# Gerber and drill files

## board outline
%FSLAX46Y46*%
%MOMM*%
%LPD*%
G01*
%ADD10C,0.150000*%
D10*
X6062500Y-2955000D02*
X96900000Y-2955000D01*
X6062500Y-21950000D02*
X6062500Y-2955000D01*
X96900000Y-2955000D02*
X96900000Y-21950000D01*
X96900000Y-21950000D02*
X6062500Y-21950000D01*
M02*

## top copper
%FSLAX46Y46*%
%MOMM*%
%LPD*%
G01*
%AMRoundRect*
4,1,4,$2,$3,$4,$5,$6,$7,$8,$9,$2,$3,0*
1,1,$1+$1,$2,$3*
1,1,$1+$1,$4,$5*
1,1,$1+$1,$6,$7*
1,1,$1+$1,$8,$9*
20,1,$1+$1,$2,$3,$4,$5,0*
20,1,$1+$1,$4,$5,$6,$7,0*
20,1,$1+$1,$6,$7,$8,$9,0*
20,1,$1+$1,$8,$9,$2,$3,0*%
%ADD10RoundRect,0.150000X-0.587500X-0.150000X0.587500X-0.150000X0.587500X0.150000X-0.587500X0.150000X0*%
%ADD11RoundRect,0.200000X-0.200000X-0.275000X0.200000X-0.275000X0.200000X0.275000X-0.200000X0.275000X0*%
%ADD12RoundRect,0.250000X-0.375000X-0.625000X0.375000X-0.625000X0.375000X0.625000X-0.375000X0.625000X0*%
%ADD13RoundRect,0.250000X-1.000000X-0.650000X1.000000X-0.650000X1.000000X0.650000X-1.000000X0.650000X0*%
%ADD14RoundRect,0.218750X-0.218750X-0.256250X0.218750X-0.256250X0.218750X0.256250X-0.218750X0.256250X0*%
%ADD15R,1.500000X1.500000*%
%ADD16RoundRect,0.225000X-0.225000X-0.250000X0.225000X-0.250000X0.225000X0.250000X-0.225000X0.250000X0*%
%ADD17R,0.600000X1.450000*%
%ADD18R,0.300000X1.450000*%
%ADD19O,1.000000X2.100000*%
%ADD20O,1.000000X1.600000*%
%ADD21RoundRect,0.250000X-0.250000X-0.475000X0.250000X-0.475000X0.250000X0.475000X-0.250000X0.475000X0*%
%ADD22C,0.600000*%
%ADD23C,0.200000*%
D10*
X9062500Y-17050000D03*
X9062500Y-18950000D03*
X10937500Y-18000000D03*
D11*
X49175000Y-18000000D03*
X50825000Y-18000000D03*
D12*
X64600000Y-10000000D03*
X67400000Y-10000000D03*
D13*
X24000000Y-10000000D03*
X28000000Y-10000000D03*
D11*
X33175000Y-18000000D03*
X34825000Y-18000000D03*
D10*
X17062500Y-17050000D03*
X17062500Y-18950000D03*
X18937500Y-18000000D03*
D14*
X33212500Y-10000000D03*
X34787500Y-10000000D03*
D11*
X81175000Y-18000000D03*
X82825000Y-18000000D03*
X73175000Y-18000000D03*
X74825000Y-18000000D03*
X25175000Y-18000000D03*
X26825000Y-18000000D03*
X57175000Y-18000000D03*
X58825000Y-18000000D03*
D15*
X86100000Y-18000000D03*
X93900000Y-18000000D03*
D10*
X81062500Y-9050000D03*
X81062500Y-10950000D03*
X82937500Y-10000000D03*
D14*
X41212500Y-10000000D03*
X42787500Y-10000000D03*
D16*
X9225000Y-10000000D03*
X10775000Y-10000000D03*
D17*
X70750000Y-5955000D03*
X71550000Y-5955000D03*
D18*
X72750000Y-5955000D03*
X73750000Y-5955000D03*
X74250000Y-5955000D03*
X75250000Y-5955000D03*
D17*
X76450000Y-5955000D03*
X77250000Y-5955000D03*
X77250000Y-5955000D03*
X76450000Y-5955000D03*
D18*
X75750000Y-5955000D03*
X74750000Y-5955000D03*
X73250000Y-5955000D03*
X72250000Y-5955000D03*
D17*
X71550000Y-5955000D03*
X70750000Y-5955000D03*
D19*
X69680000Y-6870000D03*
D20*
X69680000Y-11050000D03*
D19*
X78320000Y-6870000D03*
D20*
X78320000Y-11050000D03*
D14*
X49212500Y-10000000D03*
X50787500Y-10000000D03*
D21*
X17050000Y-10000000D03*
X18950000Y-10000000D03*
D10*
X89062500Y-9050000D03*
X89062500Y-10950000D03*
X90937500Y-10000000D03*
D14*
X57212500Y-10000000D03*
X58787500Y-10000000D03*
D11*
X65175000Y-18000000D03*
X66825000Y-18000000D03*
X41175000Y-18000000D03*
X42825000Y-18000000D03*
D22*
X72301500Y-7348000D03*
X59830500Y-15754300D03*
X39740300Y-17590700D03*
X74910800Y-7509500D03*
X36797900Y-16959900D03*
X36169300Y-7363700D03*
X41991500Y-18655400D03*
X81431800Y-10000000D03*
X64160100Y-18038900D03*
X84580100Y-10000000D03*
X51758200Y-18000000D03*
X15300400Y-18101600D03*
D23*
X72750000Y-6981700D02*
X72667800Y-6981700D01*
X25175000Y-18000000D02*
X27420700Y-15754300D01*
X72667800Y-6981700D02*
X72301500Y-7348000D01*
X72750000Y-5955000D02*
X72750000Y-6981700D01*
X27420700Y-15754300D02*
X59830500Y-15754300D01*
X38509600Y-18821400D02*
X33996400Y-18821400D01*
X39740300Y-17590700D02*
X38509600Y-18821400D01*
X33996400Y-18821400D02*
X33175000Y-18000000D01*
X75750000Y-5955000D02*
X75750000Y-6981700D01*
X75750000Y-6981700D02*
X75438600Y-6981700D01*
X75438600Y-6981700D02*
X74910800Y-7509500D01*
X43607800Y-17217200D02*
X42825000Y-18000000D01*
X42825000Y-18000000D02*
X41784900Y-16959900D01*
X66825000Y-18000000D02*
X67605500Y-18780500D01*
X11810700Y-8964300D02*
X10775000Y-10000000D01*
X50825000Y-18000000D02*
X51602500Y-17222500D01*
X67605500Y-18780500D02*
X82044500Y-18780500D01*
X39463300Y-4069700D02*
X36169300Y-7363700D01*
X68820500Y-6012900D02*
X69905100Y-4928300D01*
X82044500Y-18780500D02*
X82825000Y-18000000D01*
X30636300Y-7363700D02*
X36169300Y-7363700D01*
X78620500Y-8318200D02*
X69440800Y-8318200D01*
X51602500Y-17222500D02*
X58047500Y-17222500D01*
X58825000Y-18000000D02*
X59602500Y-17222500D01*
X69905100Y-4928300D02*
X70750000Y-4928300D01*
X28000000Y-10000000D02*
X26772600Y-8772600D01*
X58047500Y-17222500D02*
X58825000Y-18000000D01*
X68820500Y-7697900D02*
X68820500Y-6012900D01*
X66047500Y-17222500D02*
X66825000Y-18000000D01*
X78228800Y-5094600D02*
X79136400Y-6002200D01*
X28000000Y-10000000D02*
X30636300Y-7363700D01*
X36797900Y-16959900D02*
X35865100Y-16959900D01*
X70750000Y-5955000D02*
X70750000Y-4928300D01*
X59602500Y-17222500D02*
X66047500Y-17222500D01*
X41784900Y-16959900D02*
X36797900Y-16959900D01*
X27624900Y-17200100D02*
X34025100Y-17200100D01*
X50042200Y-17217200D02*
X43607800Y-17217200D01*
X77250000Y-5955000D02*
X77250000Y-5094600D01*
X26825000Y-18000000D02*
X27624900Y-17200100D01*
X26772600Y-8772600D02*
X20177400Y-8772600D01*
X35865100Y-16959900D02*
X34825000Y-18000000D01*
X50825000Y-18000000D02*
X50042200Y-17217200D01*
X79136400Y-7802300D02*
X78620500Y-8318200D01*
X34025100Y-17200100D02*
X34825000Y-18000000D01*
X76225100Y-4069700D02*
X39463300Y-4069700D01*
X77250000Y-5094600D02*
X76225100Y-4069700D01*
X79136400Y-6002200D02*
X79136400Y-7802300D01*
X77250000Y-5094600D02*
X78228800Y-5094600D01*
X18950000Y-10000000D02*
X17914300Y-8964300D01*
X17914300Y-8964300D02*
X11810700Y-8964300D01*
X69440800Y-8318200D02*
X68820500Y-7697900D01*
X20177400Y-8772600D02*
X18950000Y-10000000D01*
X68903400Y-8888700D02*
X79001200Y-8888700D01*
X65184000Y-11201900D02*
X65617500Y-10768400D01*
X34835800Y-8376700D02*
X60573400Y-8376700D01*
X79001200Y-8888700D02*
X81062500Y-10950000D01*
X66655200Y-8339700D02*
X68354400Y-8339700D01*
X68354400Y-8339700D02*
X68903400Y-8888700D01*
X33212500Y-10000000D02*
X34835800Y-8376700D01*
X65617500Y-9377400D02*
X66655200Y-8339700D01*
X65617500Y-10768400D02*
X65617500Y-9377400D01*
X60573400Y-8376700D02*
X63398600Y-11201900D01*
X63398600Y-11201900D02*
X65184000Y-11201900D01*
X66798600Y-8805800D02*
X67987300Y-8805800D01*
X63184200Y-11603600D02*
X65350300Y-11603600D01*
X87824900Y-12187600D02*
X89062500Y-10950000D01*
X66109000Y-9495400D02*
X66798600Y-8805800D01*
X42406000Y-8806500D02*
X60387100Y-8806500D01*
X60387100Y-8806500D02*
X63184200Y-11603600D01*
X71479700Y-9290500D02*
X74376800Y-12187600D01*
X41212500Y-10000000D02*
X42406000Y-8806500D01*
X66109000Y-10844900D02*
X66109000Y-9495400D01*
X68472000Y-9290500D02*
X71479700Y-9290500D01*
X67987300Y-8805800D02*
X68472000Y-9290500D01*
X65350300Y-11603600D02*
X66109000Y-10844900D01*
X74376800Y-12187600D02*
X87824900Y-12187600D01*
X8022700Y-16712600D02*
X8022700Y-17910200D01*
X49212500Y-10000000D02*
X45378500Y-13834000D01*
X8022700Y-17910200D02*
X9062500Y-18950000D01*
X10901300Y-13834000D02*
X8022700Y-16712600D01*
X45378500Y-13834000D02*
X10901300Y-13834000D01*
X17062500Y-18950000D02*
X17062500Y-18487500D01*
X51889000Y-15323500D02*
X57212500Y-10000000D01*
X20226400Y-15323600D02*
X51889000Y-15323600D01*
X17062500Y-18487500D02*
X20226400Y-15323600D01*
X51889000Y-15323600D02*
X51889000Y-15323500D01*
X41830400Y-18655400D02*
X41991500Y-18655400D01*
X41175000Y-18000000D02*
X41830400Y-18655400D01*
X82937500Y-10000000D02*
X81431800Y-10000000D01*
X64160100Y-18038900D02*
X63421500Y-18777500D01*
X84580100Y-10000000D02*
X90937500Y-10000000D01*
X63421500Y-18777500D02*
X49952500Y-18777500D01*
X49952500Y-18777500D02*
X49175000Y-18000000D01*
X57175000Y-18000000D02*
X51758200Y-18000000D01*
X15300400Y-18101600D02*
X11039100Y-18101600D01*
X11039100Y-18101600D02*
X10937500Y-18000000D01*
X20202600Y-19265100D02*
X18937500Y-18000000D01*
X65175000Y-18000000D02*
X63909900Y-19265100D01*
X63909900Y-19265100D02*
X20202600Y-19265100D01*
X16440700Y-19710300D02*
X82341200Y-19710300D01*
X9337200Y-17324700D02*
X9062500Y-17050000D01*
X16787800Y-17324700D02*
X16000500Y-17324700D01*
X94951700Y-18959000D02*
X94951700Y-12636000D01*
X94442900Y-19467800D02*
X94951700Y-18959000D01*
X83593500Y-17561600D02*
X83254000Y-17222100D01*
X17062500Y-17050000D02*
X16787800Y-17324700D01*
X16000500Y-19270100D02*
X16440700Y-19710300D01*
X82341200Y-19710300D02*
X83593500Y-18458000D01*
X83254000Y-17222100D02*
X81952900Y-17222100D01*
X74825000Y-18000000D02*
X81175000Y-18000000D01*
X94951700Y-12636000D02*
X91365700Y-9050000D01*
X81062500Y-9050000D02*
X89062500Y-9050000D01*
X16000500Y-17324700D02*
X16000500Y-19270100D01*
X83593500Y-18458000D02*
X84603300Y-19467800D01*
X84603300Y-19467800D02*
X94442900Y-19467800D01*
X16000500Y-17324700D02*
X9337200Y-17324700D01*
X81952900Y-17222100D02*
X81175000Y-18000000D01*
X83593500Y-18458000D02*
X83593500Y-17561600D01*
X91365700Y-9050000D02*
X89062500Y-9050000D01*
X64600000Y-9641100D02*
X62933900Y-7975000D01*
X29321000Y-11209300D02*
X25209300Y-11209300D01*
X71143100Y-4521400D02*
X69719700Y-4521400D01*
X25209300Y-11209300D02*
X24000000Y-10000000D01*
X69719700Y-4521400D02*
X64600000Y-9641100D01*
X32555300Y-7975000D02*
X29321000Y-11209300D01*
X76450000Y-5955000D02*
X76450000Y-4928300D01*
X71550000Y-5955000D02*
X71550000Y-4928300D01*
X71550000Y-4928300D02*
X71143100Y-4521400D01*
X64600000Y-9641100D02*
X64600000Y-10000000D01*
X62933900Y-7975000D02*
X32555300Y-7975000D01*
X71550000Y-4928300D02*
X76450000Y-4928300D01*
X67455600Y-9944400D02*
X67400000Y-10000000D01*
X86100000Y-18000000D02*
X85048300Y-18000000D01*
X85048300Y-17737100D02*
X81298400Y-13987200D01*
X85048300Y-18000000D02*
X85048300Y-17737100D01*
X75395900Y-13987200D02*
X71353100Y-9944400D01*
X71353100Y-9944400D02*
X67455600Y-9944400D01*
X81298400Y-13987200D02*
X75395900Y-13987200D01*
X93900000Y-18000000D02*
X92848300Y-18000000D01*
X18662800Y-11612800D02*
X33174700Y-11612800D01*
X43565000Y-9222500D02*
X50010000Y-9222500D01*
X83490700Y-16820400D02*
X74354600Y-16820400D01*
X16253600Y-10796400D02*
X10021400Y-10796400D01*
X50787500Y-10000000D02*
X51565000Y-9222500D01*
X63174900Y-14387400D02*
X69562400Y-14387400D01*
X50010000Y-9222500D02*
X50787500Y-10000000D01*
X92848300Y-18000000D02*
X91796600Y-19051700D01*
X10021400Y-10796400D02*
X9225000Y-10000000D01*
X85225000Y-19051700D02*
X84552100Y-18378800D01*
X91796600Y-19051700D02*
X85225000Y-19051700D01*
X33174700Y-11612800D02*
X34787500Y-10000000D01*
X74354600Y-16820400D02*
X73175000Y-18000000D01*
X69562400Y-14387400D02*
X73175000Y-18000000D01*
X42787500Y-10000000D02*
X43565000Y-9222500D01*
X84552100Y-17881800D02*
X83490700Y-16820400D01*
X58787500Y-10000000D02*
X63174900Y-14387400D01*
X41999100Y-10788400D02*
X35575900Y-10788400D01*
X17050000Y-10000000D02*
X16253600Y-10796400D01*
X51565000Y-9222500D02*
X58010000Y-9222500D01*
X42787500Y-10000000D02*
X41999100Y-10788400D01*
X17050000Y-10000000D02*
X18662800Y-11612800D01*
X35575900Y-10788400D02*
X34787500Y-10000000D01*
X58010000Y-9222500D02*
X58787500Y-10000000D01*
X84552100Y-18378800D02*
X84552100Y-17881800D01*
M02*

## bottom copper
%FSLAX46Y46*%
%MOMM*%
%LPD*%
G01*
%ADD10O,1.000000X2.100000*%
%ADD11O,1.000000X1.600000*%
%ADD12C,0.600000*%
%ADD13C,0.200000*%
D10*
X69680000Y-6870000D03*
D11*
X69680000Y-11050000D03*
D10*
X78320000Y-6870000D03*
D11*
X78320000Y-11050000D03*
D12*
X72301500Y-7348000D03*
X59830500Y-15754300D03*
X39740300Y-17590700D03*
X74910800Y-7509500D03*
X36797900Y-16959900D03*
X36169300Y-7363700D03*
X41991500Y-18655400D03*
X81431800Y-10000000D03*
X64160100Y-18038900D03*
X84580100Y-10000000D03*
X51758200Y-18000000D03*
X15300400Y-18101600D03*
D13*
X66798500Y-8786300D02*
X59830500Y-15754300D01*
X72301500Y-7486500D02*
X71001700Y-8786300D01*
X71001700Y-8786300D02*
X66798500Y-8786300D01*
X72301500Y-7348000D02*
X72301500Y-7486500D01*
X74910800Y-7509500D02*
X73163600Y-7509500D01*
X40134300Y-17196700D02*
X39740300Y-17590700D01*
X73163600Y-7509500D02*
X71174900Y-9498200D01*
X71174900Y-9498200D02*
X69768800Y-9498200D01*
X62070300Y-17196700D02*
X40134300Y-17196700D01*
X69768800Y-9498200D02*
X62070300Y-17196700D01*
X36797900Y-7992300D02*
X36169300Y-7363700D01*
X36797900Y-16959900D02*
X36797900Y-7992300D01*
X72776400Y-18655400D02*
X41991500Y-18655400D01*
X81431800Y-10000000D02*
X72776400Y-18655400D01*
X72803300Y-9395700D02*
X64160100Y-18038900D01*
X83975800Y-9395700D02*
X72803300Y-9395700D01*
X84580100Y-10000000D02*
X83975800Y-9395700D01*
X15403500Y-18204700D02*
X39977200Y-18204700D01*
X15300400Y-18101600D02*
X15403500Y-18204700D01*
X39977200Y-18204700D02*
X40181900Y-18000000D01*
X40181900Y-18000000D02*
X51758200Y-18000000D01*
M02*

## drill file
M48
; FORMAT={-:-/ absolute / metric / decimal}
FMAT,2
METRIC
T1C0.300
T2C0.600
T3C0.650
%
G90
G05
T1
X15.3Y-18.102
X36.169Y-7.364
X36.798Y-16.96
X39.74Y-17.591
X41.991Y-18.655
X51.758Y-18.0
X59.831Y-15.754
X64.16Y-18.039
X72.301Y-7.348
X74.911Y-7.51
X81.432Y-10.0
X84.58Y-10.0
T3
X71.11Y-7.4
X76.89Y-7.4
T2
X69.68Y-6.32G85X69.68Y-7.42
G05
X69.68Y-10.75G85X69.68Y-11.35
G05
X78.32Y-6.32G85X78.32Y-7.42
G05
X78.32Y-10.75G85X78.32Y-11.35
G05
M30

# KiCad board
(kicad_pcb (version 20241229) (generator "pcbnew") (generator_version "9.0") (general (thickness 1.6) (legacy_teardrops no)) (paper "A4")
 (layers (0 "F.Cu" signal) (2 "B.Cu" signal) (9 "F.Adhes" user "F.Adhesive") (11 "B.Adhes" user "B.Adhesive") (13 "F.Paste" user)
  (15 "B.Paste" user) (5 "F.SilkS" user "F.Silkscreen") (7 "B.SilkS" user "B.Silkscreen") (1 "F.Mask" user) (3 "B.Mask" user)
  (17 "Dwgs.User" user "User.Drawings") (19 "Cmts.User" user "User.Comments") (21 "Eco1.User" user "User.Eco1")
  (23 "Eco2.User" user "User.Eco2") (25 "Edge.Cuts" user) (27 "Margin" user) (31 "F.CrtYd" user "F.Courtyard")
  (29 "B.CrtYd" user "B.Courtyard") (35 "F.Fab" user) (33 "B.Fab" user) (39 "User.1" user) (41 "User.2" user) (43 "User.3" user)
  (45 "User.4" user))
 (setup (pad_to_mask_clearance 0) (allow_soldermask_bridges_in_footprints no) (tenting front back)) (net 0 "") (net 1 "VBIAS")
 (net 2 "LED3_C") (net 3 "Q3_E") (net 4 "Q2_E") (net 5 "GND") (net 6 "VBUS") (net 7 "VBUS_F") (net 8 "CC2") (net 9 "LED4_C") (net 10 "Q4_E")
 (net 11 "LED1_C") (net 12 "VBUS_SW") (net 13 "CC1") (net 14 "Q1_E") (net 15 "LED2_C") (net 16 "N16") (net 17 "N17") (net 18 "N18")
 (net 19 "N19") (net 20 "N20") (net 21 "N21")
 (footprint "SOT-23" (layer "F.Cu") (at 10 18)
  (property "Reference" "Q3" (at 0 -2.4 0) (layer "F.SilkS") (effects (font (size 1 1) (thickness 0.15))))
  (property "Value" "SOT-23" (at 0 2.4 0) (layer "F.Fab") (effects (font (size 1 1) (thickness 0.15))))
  (pad "1" smd roundrect (at -0.9375 -0.95) (size 1.475 0.6) (layers "F.Cu" "F.Mask" "F.Paste") (roundrect_rratio 0.25) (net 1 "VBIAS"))
  (pad "2" smd roundrect (at -0.9375 0.95) (size 1.475 0.6) (layers "F.Cu" "F.Mask" "F.Paste") (roundrect_rratio 0.25) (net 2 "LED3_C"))
  (pad "3" smd roundrect (at 0.9375 0) (size 1.475 0.6) (layers "F.Cu" "F.Mask" "F.Paste") (roundrect_rratio 0.25) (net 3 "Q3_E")))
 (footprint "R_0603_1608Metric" (layer "F.Cu") (at 50 18)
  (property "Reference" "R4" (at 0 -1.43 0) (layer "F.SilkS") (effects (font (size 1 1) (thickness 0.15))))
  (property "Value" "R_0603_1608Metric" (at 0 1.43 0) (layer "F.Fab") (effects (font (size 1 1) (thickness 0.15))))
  (pad "1" smd roundrect (at -0.825 0) (size 0.8 0.95) (layers "F.Cu" "F.Mask" "F.Paste") (roundrect_rratio 0.25) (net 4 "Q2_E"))
  (pad "2" smd roundrect (at 0.825 0) (size 0.8 0.95) (layers "F.Cu" "F.Mask" "F.Paste") (roundrect_rratio 0.25) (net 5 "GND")))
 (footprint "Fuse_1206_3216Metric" (layer "F.Cu") (at 66 10)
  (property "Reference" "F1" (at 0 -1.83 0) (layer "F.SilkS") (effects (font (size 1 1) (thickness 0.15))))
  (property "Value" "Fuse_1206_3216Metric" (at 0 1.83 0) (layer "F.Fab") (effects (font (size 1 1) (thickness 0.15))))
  (pad "1" smd roundrect (at -1.4 0) (size 1.25 1.75) (layers "F.Cu" "F.Mask" "F.Paste") (roundrect_rratio 0.2) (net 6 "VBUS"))
  (pad "2" smd roundrect (at 1.4 0) (size 1.25 1.75) (layers "F.Cu" "F.Mask" "F.Paste") (roundrect_rratio 0.2) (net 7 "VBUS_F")))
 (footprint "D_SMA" (layer "F.Cu") (at 26 10)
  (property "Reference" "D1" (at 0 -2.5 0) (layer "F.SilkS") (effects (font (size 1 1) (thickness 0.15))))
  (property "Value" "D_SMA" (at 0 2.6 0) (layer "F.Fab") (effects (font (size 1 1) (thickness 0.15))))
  (pad "1" smd roundrect (at -2 0) (size 2.5 1.8) (layers "F.Cu" "F.Mask" "F.Paste") (roundrect_rratio 0.1388888889) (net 6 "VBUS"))
  (pad "2" smd roundrect (at 2 0) (size 2.5 1.8) (layers "F.Cu" "F.Mask" "F.Paste") (roundrect_rratio 0.1388888889) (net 5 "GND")))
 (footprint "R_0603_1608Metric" (layer "F.Cu") (at 34 18)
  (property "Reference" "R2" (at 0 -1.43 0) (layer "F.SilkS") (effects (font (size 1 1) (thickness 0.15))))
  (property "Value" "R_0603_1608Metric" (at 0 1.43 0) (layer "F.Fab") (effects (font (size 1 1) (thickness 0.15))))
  (pad "1" smd roundrect (at -0.825 0) (size 0.8 0.95) (layers "F.Cu" "F.Mask" "F.Paste") (roundrect_rratio 0.25) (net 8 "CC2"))
  (pad "2" smd roundrect (at 0.825 0) (size 0.8 0.95) (layers "F.Cu" "F.Mask" "F.Paste") (roundrect_rratio 0.25) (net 5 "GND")))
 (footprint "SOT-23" (layer "F.Cu") (at 18 18)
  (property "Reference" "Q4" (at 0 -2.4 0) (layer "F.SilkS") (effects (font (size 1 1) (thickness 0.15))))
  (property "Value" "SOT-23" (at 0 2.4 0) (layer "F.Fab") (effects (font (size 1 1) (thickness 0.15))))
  (pad "1" smd roundrect (at -0.9375 -0.95) (size 1.475 0.6) (layers "F.Cu" "F.Mask" "F.Paste") (roundrect_rratio 0.25) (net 1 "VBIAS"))
  (pad "2" smd roundrect (at -0.9375 0.95) (size 1.475 0.6) (layers "F.Cu" "F.Mask" "F.Paste") (roundrect_rratio 0.25) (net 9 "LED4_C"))
  (pad "3" smd roundrect (at 0.9375 0) (size 1.475 0.6) (layers "F.Cu" "F.Mask" "F.Paste") (roundrect_rratio 0.25) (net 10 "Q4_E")))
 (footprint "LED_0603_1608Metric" (layer "F.Cu") (at 34 10)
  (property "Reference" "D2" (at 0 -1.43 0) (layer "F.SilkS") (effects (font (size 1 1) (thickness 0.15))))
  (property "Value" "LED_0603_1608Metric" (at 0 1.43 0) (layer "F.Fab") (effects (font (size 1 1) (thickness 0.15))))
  (pad "1" smd roundrect (at -0.7875 0) (size 0.875 0.95) (layers "F.Cu" "F.Mask" "F.Paste") (roundrect_rratio 0.25) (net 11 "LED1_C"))
  (pad "2" smd roundrect (at 0.7875 0) (size 0.875 0.95) (layers "F.Cu" "F.Mask" "F.Paste") (roundrect_rratio 0.25) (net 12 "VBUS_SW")))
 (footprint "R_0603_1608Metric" (layer "F.Cu") (at 82 18)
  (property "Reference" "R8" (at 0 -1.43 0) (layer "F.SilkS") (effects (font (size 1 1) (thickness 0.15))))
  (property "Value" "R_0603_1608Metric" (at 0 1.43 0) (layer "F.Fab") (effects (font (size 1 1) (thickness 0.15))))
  (pad "1" smd roundrect (at -0.825 0) (size 0.8 0.95) (layers "F.Cu" "F.Mask" "F.Paste") (roundrect_rratio 0.25) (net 1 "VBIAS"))
  (pad "2" smd roundrect (at 0.825 0) (size 0.8 0.95) (layers "F.Cu" "F.Mask" "F.Paste") (roundrect_rratio 0.25) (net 5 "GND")))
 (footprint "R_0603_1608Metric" (layer "F.Cu") (at 74 18)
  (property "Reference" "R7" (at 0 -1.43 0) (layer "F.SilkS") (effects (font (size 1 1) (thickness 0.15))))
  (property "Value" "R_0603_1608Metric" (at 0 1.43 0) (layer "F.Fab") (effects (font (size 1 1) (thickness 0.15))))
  (pad "1" smd roundrect (at -0.825 0) (size 0.8 0.95) (layers "F.Cu" "F.Mask" "F.Paste") (roundrect_rratio 0.25) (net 12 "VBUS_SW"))
  (pad "2" smd roundrect (at 0.825 0) (size 0.8 0.95) (layers "F.Cu" "F.Mask" "F.Paste") (roundrect_rratio 0.25) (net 1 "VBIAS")))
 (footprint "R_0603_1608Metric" (layer "F.Cu") (at 26 18)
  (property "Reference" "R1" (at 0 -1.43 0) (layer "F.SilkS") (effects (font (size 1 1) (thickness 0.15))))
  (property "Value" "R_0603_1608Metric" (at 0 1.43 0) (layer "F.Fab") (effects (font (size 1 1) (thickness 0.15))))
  (pad "1" smd roundrect (at -0.825 0) (size 0.8 0.95) (layers "F.Cu" "F.Mask" "F.Paste") (roundrect_rratio 0.25) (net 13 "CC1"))
  (pad "2" smd roundrect (at 0.825 0) (size 0.8 0.95) (layers "F.Cu" "F.Mask" "F.Paste") (roundrect_rratio 0.25) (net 5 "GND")))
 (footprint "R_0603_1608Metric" (layer "F.Cu") (at 58 18)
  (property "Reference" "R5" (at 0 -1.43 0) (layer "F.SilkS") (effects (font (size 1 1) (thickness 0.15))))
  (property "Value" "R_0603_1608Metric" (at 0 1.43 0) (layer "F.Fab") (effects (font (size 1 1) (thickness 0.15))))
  (pad "1" smd roundrect (at -0.825 0) (size 0.8 0.95) (layers "F.Cu" "F.Mask" "F.Paste") (roundrect_rratio 0.25) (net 3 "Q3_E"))
  (pad "2" smd roundrect (at 0.825 0) (size 0.8 0.95) (layers "F.Cu" "F.Mask" "F.Paste") (roundrect_rratio 0.25) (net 5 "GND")))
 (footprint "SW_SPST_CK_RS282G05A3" (layer "F.Cu") (at 90 18)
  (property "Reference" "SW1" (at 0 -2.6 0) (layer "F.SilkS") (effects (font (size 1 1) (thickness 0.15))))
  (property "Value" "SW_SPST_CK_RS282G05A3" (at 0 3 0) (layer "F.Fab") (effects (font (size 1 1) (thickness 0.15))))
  (pad "1" smd rect (at -3.9 0) (size 1.5 1.5) (layers "F.Cu" "F.Mask" "F.Paste") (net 7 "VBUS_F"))
  (pad "2" smd rect (at 3.9 0) (size 1.5 1.5) (layers "F.Cu" "F.Mask" "F.Paste") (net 12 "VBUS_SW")))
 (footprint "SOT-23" (layer "F.Cu") (at 82 10)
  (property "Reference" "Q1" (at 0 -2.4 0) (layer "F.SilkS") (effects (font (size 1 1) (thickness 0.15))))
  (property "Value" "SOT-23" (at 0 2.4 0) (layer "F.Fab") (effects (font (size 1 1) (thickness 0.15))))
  (pad "1" smd roundrect (at -0.9375 -0.95) (size 1.475 0.6) (layers "F.Cu" "F.Mask" "F.Paste") (roundrect_rratio 0.25) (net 1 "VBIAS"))
  (pad "2" smd roundrect (at -0.9375 0.95) (size 1.475 0.6) (layers "F.Cu" "F.Mask" "F.Paste") (roundrect_rratio 0.25) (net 11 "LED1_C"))
  (pad "3" smd roundrect (at 0.9375 0) (size 1.475 0.6) (layers "F.Cu" "F.Mask" "F.Paste") (roundrect_rratio 0.25) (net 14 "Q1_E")))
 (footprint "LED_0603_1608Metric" (layer "F.Cu") (at 42 10)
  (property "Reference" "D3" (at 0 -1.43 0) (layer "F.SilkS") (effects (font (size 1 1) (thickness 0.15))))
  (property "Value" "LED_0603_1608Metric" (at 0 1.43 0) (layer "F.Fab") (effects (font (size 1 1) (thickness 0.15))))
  (pad "1" smd roundrect (at -0.7875 0) (size 0.875 0.95) (layers "F.Cu" "F.Mask" "F.Paste") (roundrect_rratio 0.25) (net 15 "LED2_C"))
  (pad "2" smd roundrect (at 0.7875 0) (size 0.875 0.95) (layers "F.Cu" "F.Mask" "F.Paste") (roundrect_rratio 0.25) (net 12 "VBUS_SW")))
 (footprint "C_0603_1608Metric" (layer "F.Cu") (at 10 10)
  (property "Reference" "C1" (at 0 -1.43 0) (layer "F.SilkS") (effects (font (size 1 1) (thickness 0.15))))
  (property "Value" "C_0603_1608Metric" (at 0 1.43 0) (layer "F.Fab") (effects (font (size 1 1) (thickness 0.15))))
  (pad "1" smd roundrect (at -0.775 0) (size 0.9 0.95) (layers "F.Cu" "F.Mask" "F.Paste") (roundrect_rratio 0.25) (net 12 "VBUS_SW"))
  (pad "2" smd roundrect (at 0.775 0) (size 0.9 0.95) (layers "F.Cu" "F.Mask" "F.Paste") (roundrect_rratio 0.25) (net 5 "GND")))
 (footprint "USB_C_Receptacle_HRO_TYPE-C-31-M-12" (layer "F.Cu") (at 74 10)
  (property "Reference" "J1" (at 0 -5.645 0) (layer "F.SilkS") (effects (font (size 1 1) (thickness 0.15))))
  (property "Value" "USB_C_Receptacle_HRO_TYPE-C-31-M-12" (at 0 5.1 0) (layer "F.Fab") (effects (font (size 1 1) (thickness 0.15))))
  (pad "" np_thru_hole circle (at -2.89 -2.6) (size 0.65 0.65) (drill 0.65) (layers "*.Cu" "*.Mask"))
  (pad "" np_thru_hole circle (at 2.89 -2.6) (size 0.65 0.65) (drill 0.65) (layers "*.Cu" "*.Mask"))
  (pad "A1" smd rect (at -3.25 -4.045) (size 0.6 1.45) (layers "F.Cu" "F.Mask" "F.Paste") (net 5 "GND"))
  (pad "A4" smd rect (at -2.45 -4.045) (size 0.6 1.45) (layers "F.Cu" "F.Mask" "F.Paste") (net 6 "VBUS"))
  (pad "A5" smd rect (at -1.25 -4.045) (size 0.3 1.45) (layers "F.Cu" "F.Mask" "F.Paste") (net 13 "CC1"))
  (pad "A6" smd rect (at -0.25 -4.045) (size 0.3 1.45) (layers "F.Cu" "F.Mask" "F.Paste") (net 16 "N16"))
  (pad "A7" smd rect (at 0.25 -4.045) (size 0.3 1.45) (layers "F.Cu" "F.Mask" "F.Paste") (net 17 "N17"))
  (pad "A8" smd rect (at 1.25 -4.045) (size 0.3 1.45) (layers "F.Cu" "F.Mask" "F.Paste") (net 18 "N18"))
  (pad "A9" smd rect (at 2.45 -4.045) (size 0.6 1.45) (layers "F.Cu" "F.Mask" "F.Paste") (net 6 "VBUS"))
  (pad "A12" smd rect (at 3.25 -4.045) (size 0.6 1.45) (layers "F.Cu" "F.Mask" "F.Paste") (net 5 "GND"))
  (pad "B1" smd rect (at 3.25 -4.045) (size 0.6 1.45) (layers "F.Cu" "F.Mask" "F.Paste") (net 5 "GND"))
  (pad "B4" smd rect (at 2.45 -4.045) (size 0.6 1.45) (layers "F.Cu" "F.Mask" "F.Paste") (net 6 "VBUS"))
  (pad "B5" smd rect (at 1.75 -4.045) (size 0.3 1.45) (layers "F.Cu" "F.Mask" "F.Paste") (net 8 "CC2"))
  (pad "B6" smd rect (at 0.75 -4.045) (size 0.3 1.45) (layers "F.Cu" "F.Mask" "F.Paste") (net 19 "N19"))
  (pad "B7" smd rect (at -0.75 -4.045) (size 0.3 1.45) (layers "F.Cu" "F.Mask" "F.Paste") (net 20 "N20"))
  (pad "B8" smd rect (at -1.75 -4.045) (size 0.3 1.45) (layers "F.Cu" "F.Mask" "F.Paste") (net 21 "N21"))
  (pad "B9" smd rect (at -2.45 -4.045) (size 0.6 1.45) (layers "F.Cu" "F.Mask" "F.Paste") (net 6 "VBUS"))
  (pad "B12" smd rect (at -3.25 -4.045) (size 0.6 1.45) (layers "F.Cu" "F.Mask" "F.Paste") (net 5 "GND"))
  (pad "S1" thru_hole oval (at -4.32 -3.13) (size 1 2.1) (drill oval 0.6 1.7) (layers "*.Cu" "*.Mask") (remove_unused_layers no))
  (pad "S1" thru_hole oval (at -4.32 1.05) (size 1 1.6) (drill oval 0.6 1.2) (layers "*.Cu" "*.Mask") (remove_unused_layers no))
  (pad "S1" thru_hole oval (at 4.32 -3.13) (size 1 2.1) (drill oval 0.6 1.7) (layers "*.Cu" "*.Mask") (remove_unused_layers no))
  (pad "S1" thru_hole oval (at 4.32 1.05) (size 1 1.6) (drill oval 0.6 1.2) (layers "*.Cu" "*.Mask") (remove_unused_layers no)))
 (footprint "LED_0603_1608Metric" (layer "F.Cu") (at 50 10)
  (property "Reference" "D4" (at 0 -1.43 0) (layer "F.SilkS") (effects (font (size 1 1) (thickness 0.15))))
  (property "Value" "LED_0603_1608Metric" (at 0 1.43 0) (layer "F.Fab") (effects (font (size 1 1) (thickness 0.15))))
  (pad "1" smd roundrect (at -0.7875 0) (size 0.875 0.95) (layers "F.Cu" "F.Mask" "F.Paste") (roundrect_rratio 0.25) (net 2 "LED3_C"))
  (pad "2" smd roundrect (at 0.7875 0) (size 0.875 0.95) (layers "F.Cu" "F.Mask" "F.Paste") (roundrect_rratio 0.25) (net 12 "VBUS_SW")))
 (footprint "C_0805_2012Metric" (layer "F.Cu") (at 18 10)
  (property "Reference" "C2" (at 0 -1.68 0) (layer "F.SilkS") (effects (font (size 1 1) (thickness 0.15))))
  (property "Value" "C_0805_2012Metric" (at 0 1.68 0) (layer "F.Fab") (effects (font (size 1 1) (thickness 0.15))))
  (pad "1" smd roundrect (at -0.95 0) (size 1 1.45) (layers "F.Cu" "F.Mask" "F.Paste") (roundrect_rratio 0.25) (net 12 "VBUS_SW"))
  (pad "2" smd roundrect (at 0.95 0) (size 1 1.45) (layers "F.Cu" "F.Mask" "F.Paste") (roundrect_rratio 0.25) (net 5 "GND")))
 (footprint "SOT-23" (layer "F.Cu") (at 90 10)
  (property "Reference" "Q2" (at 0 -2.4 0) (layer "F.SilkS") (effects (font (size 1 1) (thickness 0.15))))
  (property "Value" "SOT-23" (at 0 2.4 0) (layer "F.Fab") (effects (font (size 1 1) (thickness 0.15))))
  (pad "1" smd roundrect (at -0.9375 -0.95) (size 1.475 0.6) (layers "F.Cu" "F.Mask" "F.Paste") (roundrect_rratio 0.25) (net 1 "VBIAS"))
  (pad "2" smd roundrect (at -0.9375 0.95) (size 1.475 0.6) (layers "F.Cu" "F.Mask" "F.Paste") (roundrect_rratio 0.25) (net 15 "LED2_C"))
  (pad "3" smd roundrect (at 0.9375 0) (size 1.475 0.6) (layers "F.Cu" "F.Mask" "F.Paste") (roundrect_rratio 0.25) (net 4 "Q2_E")))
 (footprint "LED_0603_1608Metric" (layer "F.Cu") (at 58 10)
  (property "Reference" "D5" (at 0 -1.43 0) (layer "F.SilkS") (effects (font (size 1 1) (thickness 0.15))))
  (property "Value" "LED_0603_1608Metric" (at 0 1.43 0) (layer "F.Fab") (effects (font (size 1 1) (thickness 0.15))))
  (pad "1" smd roundrect (at -0.7875 0) (size 0.875 0.95) (layers "F.Cu" "F.Mask" "F.Paste") (roundrect_rratio 0.25) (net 9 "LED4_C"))
  (pad "2" smd roundrect (at 0.7875 0) (size 0.875 0.95) (layers "F.Cu" "F.Mask" "F.Paste") (roundrect_rratio 0.25) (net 12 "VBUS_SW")))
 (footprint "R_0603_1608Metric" (layer "F.Cu") (at 66 18)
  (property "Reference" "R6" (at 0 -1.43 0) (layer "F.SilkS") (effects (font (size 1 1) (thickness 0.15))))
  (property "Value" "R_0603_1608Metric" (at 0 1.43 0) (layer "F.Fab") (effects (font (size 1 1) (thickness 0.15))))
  (pad "1" smd roundrect (at -0.825 0) (size 0.8 0.95) (layers "F.Cu" "F.Mask" "F.Paste") (roundrect_rratio 0.25) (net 10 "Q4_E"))
  (pad "2" smd roundrect (at 0.825 0) (size 0.8 0.95) (layers "F.Cu" "F.Mask" "F.Paste") (roundrect_rratio 0.25) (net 5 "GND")))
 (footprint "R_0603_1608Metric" (layer "F.Cu") (at 42 18)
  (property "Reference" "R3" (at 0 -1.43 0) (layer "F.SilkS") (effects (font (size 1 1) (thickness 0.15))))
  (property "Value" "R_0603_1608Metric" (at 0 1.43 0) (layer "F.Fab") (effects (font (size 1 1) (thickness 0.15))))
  (pad "1" smd roundrect (at -0.825 0) (size 0.8 0.95) (layers "F.Cu" "F.Mask" "F.Paste") (roundrect_rratio 0.25) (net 14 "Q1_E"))
  (pad "2" smd roundrect (at 0.825 0) (size 0.8 0.95) (layers "F.Cu" "F.Mask" "F.Paste") (roundrect_rratio 0.25) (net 5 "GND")))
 (gr_line (start 6.0625 2.955) (end 96.9 2.955) (stroke (width 0.15) (type default)) (layer "Edge.Cuts"))
 (gr_line (start 6.0625 21.95) (end 6.0625 2.955) (stroke (width 0.15) (type default)) (layer "Edge.Cuts"))
 (gr_line (start 96.9 2.955) (end 96.9 21.95) (stroke (width 0.15) (type default)) (layer "Edge.Cuts"))
 (gr_line (start 96.9 21.95) (end 6.0625 21.95) (stroke (width 0.15) (type default)) (layer "Edge.Cuts"))
 (segment (start 72.75 6.9817) (end 72.6678 6.9817) (width 0.2) (layer "F.Cu") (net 13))
 (segment (start 25.175 18) (end 27.4207 15.7543) (width 0.2) (layer "F.Cu") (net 13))
 (segment (start 72.6678 6.9817) (end 72.3015 7.348) (width 0.2) (layer "F.Cu") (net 13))
 (segment (start 72.75 5.955) (end 72.75 6.9817) (width 0.2) (layer "F.Cu") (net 13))
 (segment (start 27.4207 15.7543) (end 59.8305 15.7543) (width 0.2) (layer "F.Cu") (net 13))
 (via (at 72.3015 7.348) (size 0.6) (drill 0.3) (layers "F.Cu" "B.Cu") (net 13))
 (via (at 59.8305 15.7543) (size 0.6) (drill 0.3) (layers "F.Cu" "B.Cu") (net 13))
 (segment (start 66.7985 8.7863) (end 59.8305 15.7543) (width 0.2) (layer "B.Cu") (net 13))
 (segment (start 72.3015 7.4865) (end 71.0017 8.7863) (width 0.2) (layer "B.Cu") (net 13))
 (segment (start 71.0017 8.7863) (end 66.7985 8.7863) (width 0.2) (layer "B.Cu") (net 13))
 (segment (start 72.3015 7.348) (end 72.3015 7.4865) (width 0.2) (layer "B.Cu") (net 13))
 (segment (start 38.5096 18.8214) (end 33.9964 18.8214) (width 0.2) (layer "F.Cu") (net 8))
 (segment (start 39.7403 17.5907) (end 38.5096 18.8214) (width 0.2) (layer "F.Cu") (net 8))
 (segment (start 33.9964 18.8214) (end 33.175 18) (width 0.2) (layer "F.Cu") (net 8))
 (segment (start 75.75 5.955) (end 75.75 6.9817) (width 0.2) (layer "F.Cu") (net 8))
 (segment (start 75.75 6.9817) (end 75.4386 6.9817) (width 0.2) (layer "F.Cu") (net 8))
 (segment (start 75.4386 6.9817) (end 74.9108 7.5095) (width 0.2) (layer "F.Cu") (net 8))
 (via (at 39.7403 17.5907) (size 0.6) (drill 0.3) (layers "F.Cu" "B.Cu") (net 8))
 (via (at 74.9108 7.5095) (size 0.6) (drill 0.3) (layers "F.Cu" "B.Cu") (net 8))
 (segment (start 74.9108 7.5095) (end 73.1636 7.5095) (width 0.2) (layer "B.Cu") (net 8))
 (segment (start 40.1343 17.1967) (end 39.7403 17.5907) (width 0.2) (layer "B.Cu") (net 8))
 (segment (start 73.1636 7.5095) (end 71.1749 9.4982) (width 0.2) (layer "B.Cu") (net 8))
 (segment (start 71.1749 9.4982) (end 69.7688 9.4982) (width 0.2) (layer "B.Cu") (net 8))
 (segment (start 62.0703 17.1967) (end 40.1343 17.1967) (width 0.2) (layer "B.Cu") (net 8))
 (segment (start 69.7688 9.4982) (end 62.0703 17.1967) (width 0.2) (layer "B.Cu") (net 8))
 (segment (start 43.6078 17.2172) (end 42.825 18) (width 0.2) (layer "F.Cu") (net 5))
 (segment (start 42.825 18) (end 41.7849 16.9599) (width 0.2) (layer "F.Cu") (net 5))
 (segment (start 66.825 18) (end 67.6055 18.7805) (width 0.2) (layer "F.Cu") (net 5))
 (segment (start 11.8107 8.9643) (end 10.775 10) (width 0.2) (layer "F.Cu") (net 5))
 (segment (start 50.825 18) (end 51.6025 17.2225) (width 0.2) (layer "F.Cu") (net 5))
 (segment (start 67.6055 18.7805) (end 82.0445 18.7805) (width 0.2) (layer "F.Cu") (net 5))
 (segment (start 39.4633 4.0697) (end 36.1693 7.3637) (width 0.2) (layer "F.Cu") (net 5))
 (segment (start 68.8205 6.0129) (end 69.9051 4.9283) (width 0.2) (layer "F.Cu") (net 5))
 (segment (start 82.0445 18.7805) (end 82.825 18) (width 0.2) (layer "F.Cu") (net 5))
 (segment (start 30.6363 7.3637) (end 36.1693 7.3637) (width 0.2) (layer "F.Cu") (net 5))
 (segment (start 78.6205 8.3182) (end 69.4408 8.3182) (width 0.2) (layer "F.Cu") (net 5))
 (segment (start 51.6025 17.2225) (end 58.0475 17.2225) (width 0.2) (layer "F.Cu") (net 5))
 (segment (start 58.825 18) (end 59.6025 17.2225) (width 0.2) (layer "F.Cu") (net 5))
 (segment (start 69.9051 4.9283) (end 70.75 4.9283) (width 0.2) (layer "F.Cu") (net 5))
 (segment (start 28 10) (end 26.7726 8.7726) (width 0.2) (layer "F.Cu") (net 5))
 (segment (start 58.0475 17.2225) (end 58.825 18) (width 0.2) (layer "F.Cu") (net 5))
 (segment (start 68.8205 7.6979) (end 68.8205 6.0129) (width 0.2) (layer "F.Cu") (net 5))
 (segment (start 66.0475 17.2225) (end 66.825 18) (width 0.2) (layer "F.Cu") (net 5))
 (segment (start 78.2288 5.0946) (end 79.1364 6.0022) (width 0.2) (layer "F.Cu") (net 5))
 (segment (start 28 10) (end 30.6363 7.3637) (width 0.2) (layer "F.Cu") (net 5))
 (segment (start 36.7979 16.9599) (end 35.8651 16.9599) (width 0.2) (layer "F.Cu") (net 5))
 (segment (start 70.75 5.955) (end 70.75 4.9283) (width 0.2) (layer "F.Cu") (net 5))
 (segment (start 59.6025 17.2225) (end 66.0475 17.2225) (width 0.2) (layer "F.Cu") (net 5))
 (segment (start 41.7849 16.9599) (end 36.7979 16.9599) (width 0.2) (layer "F.Cu") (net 5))
 (segment (start 27.6249 17.2001) (end 34.0251 17.2001) (width 0.2) (layer "F.Cu") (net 5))
 (segment (start 50.0422 17.2172) (end 43.6078 17.2172) (width 0.2) (layer "F.Cu") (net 5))
 (segment (start 77.25 5.955) (end 77.25 5.0946) (width 0.2) (layer "F.Cu") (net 5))
 (segment (start 26.825 18) (end 27.6249 17.2001) (width 0.2) (layer "F.Cu") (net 5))
 (segment (start 26.7726 8.7726) (end 20.1774 8.7726) (width 0.2) (layer "F.Cu") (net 5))
 (segment (start 35.8651 16.9599) (end 34.825 18) (width 0.2) (layer "F.Cu") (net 5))
 (segment (start 50.825 18) (end 50.0422 17.2172) (width 0.2) (layer "F.Cu") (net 5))
 (segment (start 79.1364 7.8023) (end 78.6205 8.3182) (width 0.2) (layer "F.Cu") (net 5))
 (segment (start 34.0251 17.2001) (end 34.825 18) (width 0.2) (layer "F.Cu") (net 5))
 (segment (start 76.2251 4.0697) (end 39.4633 4.0697) (width 0.2) (layer "F.Cu") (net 5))
 (segment (start 77.25 5.0946) (end 76.2251 4.0697) (width 0.2) (layer "F.Cu") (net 5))
 (segment (start 79.1364 6.0022) (end 79.1364 7.8023) (width 0.2) (layer "F.Cu") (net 5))
 (segment (start 77.25 5.0946) (end 78.2288 5.0946) (width 0.2) (layer "F.Cu") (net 5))
 (segment (start 18.95 10) (end 17.9143 8.9643) (width 0.2) (layer "F.Cu") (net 5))
 (segment (start 17.9143 8.9643) (end 11.8107 8.9643) (width 0.2) (layer "F.Cu") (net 5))
 (segment (start 69.4408 8.3182) (end 68.8205 7.6979) (width 0.2) (layer "F.Cu") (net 5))
 (segment (start 20.1774 8.7726) (end 18.95 10) (width 0.2) (layer "F.Cu") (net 5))
 (via (at 36.7979 16.9599) (size 0.6) (drill 0.3) (layers "F.Cu" "B.Cu") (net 5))
 (via (at 36.1693 7.3637) (size 0.6) (drill 0.3) (layers "F.Cu" "B.Cu") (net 5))
 (segment (start 36.7979 7.9923) (end 36.1693 7.3637) (width 0.2) (layer "B.Cu") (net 5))
 (segment (start 36.7979 16.9599) (end 36.7979 7.9923) (width 0.2) (layer "B.Cu") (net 5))
 (segment (start 68.9034 8.8887) (end 79.0012 8.8887) (width 0.2) (layer "F.Cu") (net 11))
 (segment (start 65.184 11.2019) (end 65.6175 10.7684) (width 0.2) (layer "F.Cu") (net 11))
 (segment (start 34.8358 8.3767) (end 60.5734 8.3767) (width 0.2) (layer "F.Cu") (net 11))
 (segment (start 79.0012 8.8887) (end 81.0625 10.95) (width 0.2) (layer "F.Cu") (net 11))
 (segment (start 66.6552 8.3397) (end 68.3544 8.3397) (width 0.2) (layer "F.Cu") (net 11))
 (segment (start 68.3544 8.3397) (end 68.9034 8.8887) (width 0.2) (layer "F.Cu") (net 11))
 (segment (start 33.2125 10) (end 34.8358 8.3767) (width 0.2) (layer "F.Cu") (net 11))
 (segment (start 65.6175 9.3774) (end 66.6552 8.3397) (width 0.2) (layer "F.Cu") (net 11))
 (segment (start 65.6175 10.7684) (end 65.6175 9.3774) (width 0.2) (layer "F.Cu") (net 11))
 (segment (start 60.5734 8.3767) (end 63.3986 11.2019) (width 0.2) (layer "F.Cu") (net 11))
 (segment (start 63.3986 11.2019) (end 65.184 11.2019) (width 0.2) (layer "F.Cu") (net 11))
 (segment (start 66.7986 8.8058) (end 67.9873 8.8058) (width 0.2) (layer "F.Cu") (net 15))
 (segment (start 63.1842 11.6036) (end 65.3503 11.6036) (width 0.2) (layer "F.Cu") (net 15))
 (segment (start 87.8249 12.1876) (end 89.0625 10.95) (width 0.2) (layer "F.Cu") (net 15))
 (segment (start 66.109 9.4954) (end 66.7986 8.8058) (width 0.2) (layer "F.Cu") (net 15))
 (segment (start 42.406 8.8065) (end 60.3871 8.8065) (width 0.2) (layer "F.Cu") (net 15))
 (segment (start 60.3871 8.8065) (end 63.1842 11.6036) (width 0.2) (layer "F.Cu") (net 15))
 (segment (start 71.4797 9.2905) (end 74.3768 12.1876) (width 0.2) (layer "F.Cu") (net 15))
 (segment (start 41.2125 10) (end 42.406 8.8065) (width 0.2) (layer "F.Cu") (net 15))
 (segment (start 66.109 10.8449) (end 66.109 9.4954) (width 0.2) (layer "F.Cu") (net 15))
 (segment (start 68.472 9.2905) (end 71.4797 9.2905) (width 0.2) (layer "F.Cu") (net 15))
 (segment (start 67.9873 8.8058) (end 68.472 9.2905) (width 0.2) (layer "F.Cu") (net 15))
 (segment (start 65.3503 11.6036) (end 66.109 10.8449) (width 0.2) (layer "F.Cu") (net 15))
 (segment (start 74.3768 12.1876) (end 87.8249 12.1876) (width 0.2) (layer "F.Cu") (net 15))
 (segment (start 8.0227 16.7126) (end 8.0227 17.9102) (width 0.2) (layer "F.Cu") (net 2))
 (segment (start 49.2125 10) (end 45.3785 13.834) (width 0.2) (layer "F.Cu") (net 2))
 (segment (start 8.0227 17.9102) (end 9.0625 18.95) (width 0.2) (layer "F.Cu") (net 2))
 (segment (start 10.9013 13.834) (end 8.0227 16.7126) (width 0.2) (layer "F.Cu") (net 2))
 (segment (start 45.3785 13.834) (end 10.9013 13.834) (width 0.2) (layer "F.Cu") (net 2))
 (segment (start 17.0625 18.95) (end 17.0625 18.4875) (width 0.2) (layer "F.Cu") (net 9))
 (segment (start 51.889 15.3235) (end 57.2125 10) (width 0.2) (layer "F.Cu") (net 9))
 (segment (start 20.2264 15.3236) (end 51.889 15.3236) (width 0.2) (layer "F.Cu") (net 9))
 (segment (start 17.0625 18.4875) (end 20.2264 15.3236) (width 0.2) (layer "F.Cu") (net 9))
 (segment (start 51.889 15.3236) (end 51.889 15.3235) (width 0.2) (layer "F.Cu") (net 9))
 (segment (start 41.8304 18.6554) (end 41.9915 18.6554) (width 0.2) (layer "F.Cu") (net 14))
 (segment (start 41.175 18) (end 41.8304 18.6554) (width 0.2) (layer "F.Cu") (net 14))
 (segment (start 82.9375 10) (end 81.4318 10) (width 0.2) (layer "F.Cu") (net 14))
 (via (at 41.9915 18.6554) (size 0.6) (drill 0.3) (layers "F.Cu" "B.Cu") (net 14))
 (via (at 81.4318 10) (size 0.6) (drill 0.3) (layers "F.Cu" "B.Cu") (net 14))
 (segment (start 72.7764 18.6554) (end 41.9915 18.6554) (width 0.2) (layer "B.Cu") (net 14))
 (segment (start 81.4318 10) (end 72.7764 18.6554) (width 0.2) (layer "B.Cu") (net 14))
 (segment (start 64.1601 18.0389) (end 63.4215 18.7775) (width 0.2) (layer "F.Cu") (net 4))
 (segment (start 84.5801 10) (end 90.9375 10) (width 0.2) (layer "F.Cu") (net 4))
 (segment (start 63.4215 18.7775) (end 49.9525 18.7775) (width 0.2) (layer "F.Cu") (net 4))
 (segment (start 49.9525 18.7775) (end 49.175 18) (width 0.2) (layer "F.Cu") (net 4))
 (via (at 64.1601 18.0389) (size 0.6) (drill 0.3) (layers "F.Cu" "B.Cu") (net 4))
 (via (at 84.5801 10) (size 0.6) (drill 0.3) (layers "F.Cu" "B.Cu") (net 4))
 (segment (start 72.8033 9.3957) (end 64.1601 18.0389) (width 0.2) (layer "B.Cu") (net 4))
 (segment (start 83.9758 9.3957) (end 72.8033 9.3957) (width 0.2) (layer "B.Cu") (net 4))
 (segment (start 84.5801 10) (end 83.9758 9.3957) (width 0.2) (layer "B.Cu") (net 4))
 (segment (start 57.175 18) (end 51.7582 18) (width 0.2) (layer "F.Cu") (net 3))
 (segment (start 15.3004 18.1016) (end 11.0391 18.1016) (width 0.2) (layer "F.Cu") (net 3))
 (segment (start 11.0391 18.1016) (end 10.9375 18) (width 0.2) (layer "F.Cu") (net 3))
 (via (at 51.7582 18) (size 0.6) (drill 0.3) (layers "F.Cu" "B.Cu") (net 3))
 (via (at 15.3004 18.1016) (size 0.6) (drill 0.3) (layers "F.Cu" "B.Cu") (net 3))
 (segment (start 15.4035 18.2047) (end 39.9772 18.2047) (width 0.2) (layer "B.Cu") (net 3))
 (segment (start 15.3004 18.1016) (end 15.4035 18.2047) (width 0.2) (layer "B.Cu") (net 3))
 (segment (start 39.9772 18.2047) (end 40.1819 18) (width 0.2) (layer "B.Cu") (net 3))
 (segment (start 40.1819 18) (end 51.7582 18) (width 0.2) (layer "B.Cu") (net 3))
 (segment (start 20.2026 19.2651) (end 18.9375 18) (width 0.2) (layer "F.Cu") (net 10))
 (segment (start 65.175 18) (end 63.9099 19.2651) (width 0.2) (layer "F.Cu") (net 10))
 (segment (start 63.9099 19.2651) (end 20.2026 19.2651) (width 0.2) (layer "F.Cu") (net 10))
 (segment (start 16.4407 19.7103) (end 82.3412 19.7103) (width 0.2) (layer "F.Cu") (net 1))
 (segment (start 9.3372 17.3247) (end 9.0625 17.05) (width 0.2) (layer "F.Cu") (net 1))
 (segment (start 16.7878 17.3247) (end 16.0005 17.3247) (width 0.2) (layer "F.Cu") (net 1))
 (segment (start 94.9517 18.959) (end 94.9517 12.636) (width 0.2) (layer "F.Cu") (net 1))
 (segment (start 94.4429 19.4678) (end 94.9517 18.959) (width 0.2) (layer "F.Cu") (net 1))
 (segment (start 83.5935 17.5616) (end 83.254 17.2221) (width 0.2) (layer "F.Cu") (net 1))
 (segment (start 17.0625 17.05) (end 16.7878 17.3247) (width 0.2) (layer "F.Cu") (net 1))
 (segment (start 16.0005 19.2701) (end 16.4407 19.7103) (width 0.2) (layer "F.Cu") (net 1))
 (segment (start 82.3412 19.7103) (end 83.5935 18.458) (width 0.2) (layer "F.Cu") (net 1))
 (segment (start 83.254 17.2221) (end 81.9529 17.2221) (width 0.2) (layer "F.Cu") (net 1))
 (segment (start 74.825 18) (end 81.175 18) (width 0.2) (layer "F.Cu") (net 1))
 (segment (start 94.9517 12.636) (end 91.3657 9.05) (width 0.2) (layer "F.Cu") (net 1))
 (segment (start 81.0625 9.05) (end 89.0625 9.05) (width 0.2) (layer "F.Cu") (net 1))
 (segment (start 16.0005 17.3247) (end 16.0005 19.2701) (width 0.2) (layer "F.Cu") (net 1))
 (segment (start 83.5935 18.458) (end 84.6033 19.4678) (width 0.2) (layer "F.Cu") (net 1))
 (segment (start 84.6033 19.4678) (end 94.4429 19.4678) (width 0.2) (layer "F.Cu") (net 1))
 (segment (start 16.0005 17.3247) (end 9.3372 17.3247) (width 0.2) (layer "F.Cu") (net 1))
 (segment (start 81.9529 17.2221) (end 81.175 18) (width 0.2) (layer "F.Cu") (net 1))
 (segment (start 83.5935 18.458) (end 83.5935 17.5616) (width 0.2) (layer "F.Cu") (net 1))
 (segment (start 91.3657 9.05) (end 89.0625 9.05) (width 0.2) (layer "F.Cu") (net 1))
 (segment (start 64.6 9.6411) (end 62.9339 7.975) (width 0.2) (layer "F.Cu") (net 6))
 (segment (start 29.321 11.2093) (end 25.2093 11.2093) (width 0.2) (layer "F.Cu") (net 6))
 (segment (start 71.1431 4.5214) (end 69.7197 4.5214) (width 0.2) (layer "F.Cu") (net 6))
 (segment (start 25.2093 11.2093) (end 24 10) (width 0.2) (layer "F.Cu") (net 6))
 (segment (start 69.7197 4.5214) (end 64.6 9.6411) (width 0.2) (layer "F.Cu") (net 6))
 (segment (start 32.5553 7.975) (end 29.321 11.2093) (width 0.2) (layer "F.Cu") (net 6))
 (segment (start 76.45 5.955) (end 76.45 4.9283) (width 0.2) (layer "F.Cu") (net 6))
 (segment (start 71.55 5.955) (end 71.55 4.9283) (width 0.2) (layer "F.Cu") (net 6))
 (segment (start 71.55 4.9283) (end 71.1431 4.5214) (width 0.2) (layer "F.Cu") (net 6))
 (segment (start 64.6 9.6411) (end 64.6 10) (width 0.2) (layer "F.Cu") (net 6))
 (segment (start 62.9339 7.975) (end 32.5553 7.975) (width 0.2) (layer "F.Cu") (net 6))
 (segment (start 71.55 4.9283) (end 76.45 4.9283) (width 0.2) (layer "F.Cu") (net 6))
 (segment (start 67.4556 9.9444) (end 67.4 10) (width 0.2) (layer "F.Cu") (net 7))
 (segment (start 86.1 18) (end 85.0483 18) (width 0.2) (layer "F.Cu") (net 7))
 (segment (start 85.0483 17.7371) (end 81.2984 13.9872) (width 0.2) (layer "F.Cu") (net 7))
 (segment (start 85.0483 18) (end 85.0483 17.7371) (width 0.2) (layer "F.Cu") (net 7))
 (segment (start 75.3959 13.9872) (end 71.3531 9.9444) (width 0.2) (layer "F.Cu") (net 7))
 (segment (start 71.3531 9.9444) (end 67.4556 9.9444) (width 0.2) (layer "F.Cu") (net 7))
 (segment (start 81.2984 13.9872) (end 75.3959 13.9872) (width 0.2) (layer "F.Cu") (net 7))
 (segment (start 93.9 18) (end 92.8483 18) (width 0.2) (layer "F.Cu") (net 12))
 (segment (start 18.6628 11.6128) (end 33.1747 11.6128) (width 0.2) (layer "F.Cu") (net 12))
 (segment (start 43.565 9.2225) (end 50.01 9.2225) (width 0.2) (layer "F.Cu") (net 12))
 (segment (start 83.4907 16.8204) (end 74.3546 16.8204) (width 0.2) (layer "F.Cu") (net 12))
 (segment (start 16.2536 10.7964) (end 10.0214 10.7964) (width 0.2) (layer "F.Cu") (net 12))
 (segment (start 50.7875 10) (end 51.565 9.2225) (width 0.2) (layer "F.Cu") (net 12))
 (segment (start 63.1749 14.3874) (end 69.5624 14.3874) (width 0.2) (layer "F.Cu") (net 12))
 (segment (start 50.01 9.2225) (end 50.7875 10) (width 0.2) (layer "F.Cu") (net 12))
 (segment (start 92.8483 18) (end 91.7966 19.0517) (width 0.2) (layer "F.Cu") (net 12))
 (segment (start 10.0214 10.7964) (end 9.225 10) (width 0.2) (layer "F.Cu") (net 12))
 (segment (start 85.225 19.0517) (end 84.5521 18.3788) (width 0.2) (layer "F.Cu") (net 12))
 (segment (start 91.7966 19.0517) (end 85.225 19.0517) (width 0.2) (layer "F.Cu") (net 12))
 (segment (start 33.1747 11.6128) (end 34.7875 10) (width 0.2) (layer "F.Cu") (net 12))
 (segment (start 74.3546 16.8204) (end 73.175 18) (width 0.2) (layer "F.Cu") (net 12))
 (segment (start 69.5624 14.3874) (end 73.175 18) (width 0.2) (layer "F.Cu") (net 12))
 (segment (start 42.7875 10) (end 43.565 9.2225) (width 0.2) (layer "F.Cu") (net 12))
 (segment (start 84.5521 17.8818) (end 83.4907 16.8204) (width 0.2) (layer "F.Cu") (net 12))
 (segment (start 58.7875 10) (end 63.1749 14.3874) (width 0.2) (layer "F.Cu") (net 12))
 (segment (start 41.9991 10.7884) (end 35.5759 10.7884) (width 0.2) (layer "F.Cu") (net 12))
 (segment (start 17.05 10) (end 16.2536 10.7964) (width 0.2) (layer "F.Cu") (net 12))
 (segment (start 51.565 9.2225) (end 58.01 9.2225) (width 0.2) (layer "F.Cu") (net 12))
 (segment (start 42.7875 10) (end 41.9991 10.7884) (width 0.2) (layer "F.Cu") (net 12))
 (segment (start 17.05 10) (end 18.6628 11.6128) (width 0.2) (layer "F.Cu") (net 12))
 (segment (start 35.5759 10.7884) (end 34.7875 10) (width 0.2) (layer "F.Cu") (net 12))
 (segment (start 58.01 9.2225) (end 58.7875 10) (width 0.2) (layer "F.Cu") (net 12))
 (segment (start 84.5521 18.3788) (end 84.5521 17.8818) (width 0.2) (layer "F.Cu") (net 12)))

